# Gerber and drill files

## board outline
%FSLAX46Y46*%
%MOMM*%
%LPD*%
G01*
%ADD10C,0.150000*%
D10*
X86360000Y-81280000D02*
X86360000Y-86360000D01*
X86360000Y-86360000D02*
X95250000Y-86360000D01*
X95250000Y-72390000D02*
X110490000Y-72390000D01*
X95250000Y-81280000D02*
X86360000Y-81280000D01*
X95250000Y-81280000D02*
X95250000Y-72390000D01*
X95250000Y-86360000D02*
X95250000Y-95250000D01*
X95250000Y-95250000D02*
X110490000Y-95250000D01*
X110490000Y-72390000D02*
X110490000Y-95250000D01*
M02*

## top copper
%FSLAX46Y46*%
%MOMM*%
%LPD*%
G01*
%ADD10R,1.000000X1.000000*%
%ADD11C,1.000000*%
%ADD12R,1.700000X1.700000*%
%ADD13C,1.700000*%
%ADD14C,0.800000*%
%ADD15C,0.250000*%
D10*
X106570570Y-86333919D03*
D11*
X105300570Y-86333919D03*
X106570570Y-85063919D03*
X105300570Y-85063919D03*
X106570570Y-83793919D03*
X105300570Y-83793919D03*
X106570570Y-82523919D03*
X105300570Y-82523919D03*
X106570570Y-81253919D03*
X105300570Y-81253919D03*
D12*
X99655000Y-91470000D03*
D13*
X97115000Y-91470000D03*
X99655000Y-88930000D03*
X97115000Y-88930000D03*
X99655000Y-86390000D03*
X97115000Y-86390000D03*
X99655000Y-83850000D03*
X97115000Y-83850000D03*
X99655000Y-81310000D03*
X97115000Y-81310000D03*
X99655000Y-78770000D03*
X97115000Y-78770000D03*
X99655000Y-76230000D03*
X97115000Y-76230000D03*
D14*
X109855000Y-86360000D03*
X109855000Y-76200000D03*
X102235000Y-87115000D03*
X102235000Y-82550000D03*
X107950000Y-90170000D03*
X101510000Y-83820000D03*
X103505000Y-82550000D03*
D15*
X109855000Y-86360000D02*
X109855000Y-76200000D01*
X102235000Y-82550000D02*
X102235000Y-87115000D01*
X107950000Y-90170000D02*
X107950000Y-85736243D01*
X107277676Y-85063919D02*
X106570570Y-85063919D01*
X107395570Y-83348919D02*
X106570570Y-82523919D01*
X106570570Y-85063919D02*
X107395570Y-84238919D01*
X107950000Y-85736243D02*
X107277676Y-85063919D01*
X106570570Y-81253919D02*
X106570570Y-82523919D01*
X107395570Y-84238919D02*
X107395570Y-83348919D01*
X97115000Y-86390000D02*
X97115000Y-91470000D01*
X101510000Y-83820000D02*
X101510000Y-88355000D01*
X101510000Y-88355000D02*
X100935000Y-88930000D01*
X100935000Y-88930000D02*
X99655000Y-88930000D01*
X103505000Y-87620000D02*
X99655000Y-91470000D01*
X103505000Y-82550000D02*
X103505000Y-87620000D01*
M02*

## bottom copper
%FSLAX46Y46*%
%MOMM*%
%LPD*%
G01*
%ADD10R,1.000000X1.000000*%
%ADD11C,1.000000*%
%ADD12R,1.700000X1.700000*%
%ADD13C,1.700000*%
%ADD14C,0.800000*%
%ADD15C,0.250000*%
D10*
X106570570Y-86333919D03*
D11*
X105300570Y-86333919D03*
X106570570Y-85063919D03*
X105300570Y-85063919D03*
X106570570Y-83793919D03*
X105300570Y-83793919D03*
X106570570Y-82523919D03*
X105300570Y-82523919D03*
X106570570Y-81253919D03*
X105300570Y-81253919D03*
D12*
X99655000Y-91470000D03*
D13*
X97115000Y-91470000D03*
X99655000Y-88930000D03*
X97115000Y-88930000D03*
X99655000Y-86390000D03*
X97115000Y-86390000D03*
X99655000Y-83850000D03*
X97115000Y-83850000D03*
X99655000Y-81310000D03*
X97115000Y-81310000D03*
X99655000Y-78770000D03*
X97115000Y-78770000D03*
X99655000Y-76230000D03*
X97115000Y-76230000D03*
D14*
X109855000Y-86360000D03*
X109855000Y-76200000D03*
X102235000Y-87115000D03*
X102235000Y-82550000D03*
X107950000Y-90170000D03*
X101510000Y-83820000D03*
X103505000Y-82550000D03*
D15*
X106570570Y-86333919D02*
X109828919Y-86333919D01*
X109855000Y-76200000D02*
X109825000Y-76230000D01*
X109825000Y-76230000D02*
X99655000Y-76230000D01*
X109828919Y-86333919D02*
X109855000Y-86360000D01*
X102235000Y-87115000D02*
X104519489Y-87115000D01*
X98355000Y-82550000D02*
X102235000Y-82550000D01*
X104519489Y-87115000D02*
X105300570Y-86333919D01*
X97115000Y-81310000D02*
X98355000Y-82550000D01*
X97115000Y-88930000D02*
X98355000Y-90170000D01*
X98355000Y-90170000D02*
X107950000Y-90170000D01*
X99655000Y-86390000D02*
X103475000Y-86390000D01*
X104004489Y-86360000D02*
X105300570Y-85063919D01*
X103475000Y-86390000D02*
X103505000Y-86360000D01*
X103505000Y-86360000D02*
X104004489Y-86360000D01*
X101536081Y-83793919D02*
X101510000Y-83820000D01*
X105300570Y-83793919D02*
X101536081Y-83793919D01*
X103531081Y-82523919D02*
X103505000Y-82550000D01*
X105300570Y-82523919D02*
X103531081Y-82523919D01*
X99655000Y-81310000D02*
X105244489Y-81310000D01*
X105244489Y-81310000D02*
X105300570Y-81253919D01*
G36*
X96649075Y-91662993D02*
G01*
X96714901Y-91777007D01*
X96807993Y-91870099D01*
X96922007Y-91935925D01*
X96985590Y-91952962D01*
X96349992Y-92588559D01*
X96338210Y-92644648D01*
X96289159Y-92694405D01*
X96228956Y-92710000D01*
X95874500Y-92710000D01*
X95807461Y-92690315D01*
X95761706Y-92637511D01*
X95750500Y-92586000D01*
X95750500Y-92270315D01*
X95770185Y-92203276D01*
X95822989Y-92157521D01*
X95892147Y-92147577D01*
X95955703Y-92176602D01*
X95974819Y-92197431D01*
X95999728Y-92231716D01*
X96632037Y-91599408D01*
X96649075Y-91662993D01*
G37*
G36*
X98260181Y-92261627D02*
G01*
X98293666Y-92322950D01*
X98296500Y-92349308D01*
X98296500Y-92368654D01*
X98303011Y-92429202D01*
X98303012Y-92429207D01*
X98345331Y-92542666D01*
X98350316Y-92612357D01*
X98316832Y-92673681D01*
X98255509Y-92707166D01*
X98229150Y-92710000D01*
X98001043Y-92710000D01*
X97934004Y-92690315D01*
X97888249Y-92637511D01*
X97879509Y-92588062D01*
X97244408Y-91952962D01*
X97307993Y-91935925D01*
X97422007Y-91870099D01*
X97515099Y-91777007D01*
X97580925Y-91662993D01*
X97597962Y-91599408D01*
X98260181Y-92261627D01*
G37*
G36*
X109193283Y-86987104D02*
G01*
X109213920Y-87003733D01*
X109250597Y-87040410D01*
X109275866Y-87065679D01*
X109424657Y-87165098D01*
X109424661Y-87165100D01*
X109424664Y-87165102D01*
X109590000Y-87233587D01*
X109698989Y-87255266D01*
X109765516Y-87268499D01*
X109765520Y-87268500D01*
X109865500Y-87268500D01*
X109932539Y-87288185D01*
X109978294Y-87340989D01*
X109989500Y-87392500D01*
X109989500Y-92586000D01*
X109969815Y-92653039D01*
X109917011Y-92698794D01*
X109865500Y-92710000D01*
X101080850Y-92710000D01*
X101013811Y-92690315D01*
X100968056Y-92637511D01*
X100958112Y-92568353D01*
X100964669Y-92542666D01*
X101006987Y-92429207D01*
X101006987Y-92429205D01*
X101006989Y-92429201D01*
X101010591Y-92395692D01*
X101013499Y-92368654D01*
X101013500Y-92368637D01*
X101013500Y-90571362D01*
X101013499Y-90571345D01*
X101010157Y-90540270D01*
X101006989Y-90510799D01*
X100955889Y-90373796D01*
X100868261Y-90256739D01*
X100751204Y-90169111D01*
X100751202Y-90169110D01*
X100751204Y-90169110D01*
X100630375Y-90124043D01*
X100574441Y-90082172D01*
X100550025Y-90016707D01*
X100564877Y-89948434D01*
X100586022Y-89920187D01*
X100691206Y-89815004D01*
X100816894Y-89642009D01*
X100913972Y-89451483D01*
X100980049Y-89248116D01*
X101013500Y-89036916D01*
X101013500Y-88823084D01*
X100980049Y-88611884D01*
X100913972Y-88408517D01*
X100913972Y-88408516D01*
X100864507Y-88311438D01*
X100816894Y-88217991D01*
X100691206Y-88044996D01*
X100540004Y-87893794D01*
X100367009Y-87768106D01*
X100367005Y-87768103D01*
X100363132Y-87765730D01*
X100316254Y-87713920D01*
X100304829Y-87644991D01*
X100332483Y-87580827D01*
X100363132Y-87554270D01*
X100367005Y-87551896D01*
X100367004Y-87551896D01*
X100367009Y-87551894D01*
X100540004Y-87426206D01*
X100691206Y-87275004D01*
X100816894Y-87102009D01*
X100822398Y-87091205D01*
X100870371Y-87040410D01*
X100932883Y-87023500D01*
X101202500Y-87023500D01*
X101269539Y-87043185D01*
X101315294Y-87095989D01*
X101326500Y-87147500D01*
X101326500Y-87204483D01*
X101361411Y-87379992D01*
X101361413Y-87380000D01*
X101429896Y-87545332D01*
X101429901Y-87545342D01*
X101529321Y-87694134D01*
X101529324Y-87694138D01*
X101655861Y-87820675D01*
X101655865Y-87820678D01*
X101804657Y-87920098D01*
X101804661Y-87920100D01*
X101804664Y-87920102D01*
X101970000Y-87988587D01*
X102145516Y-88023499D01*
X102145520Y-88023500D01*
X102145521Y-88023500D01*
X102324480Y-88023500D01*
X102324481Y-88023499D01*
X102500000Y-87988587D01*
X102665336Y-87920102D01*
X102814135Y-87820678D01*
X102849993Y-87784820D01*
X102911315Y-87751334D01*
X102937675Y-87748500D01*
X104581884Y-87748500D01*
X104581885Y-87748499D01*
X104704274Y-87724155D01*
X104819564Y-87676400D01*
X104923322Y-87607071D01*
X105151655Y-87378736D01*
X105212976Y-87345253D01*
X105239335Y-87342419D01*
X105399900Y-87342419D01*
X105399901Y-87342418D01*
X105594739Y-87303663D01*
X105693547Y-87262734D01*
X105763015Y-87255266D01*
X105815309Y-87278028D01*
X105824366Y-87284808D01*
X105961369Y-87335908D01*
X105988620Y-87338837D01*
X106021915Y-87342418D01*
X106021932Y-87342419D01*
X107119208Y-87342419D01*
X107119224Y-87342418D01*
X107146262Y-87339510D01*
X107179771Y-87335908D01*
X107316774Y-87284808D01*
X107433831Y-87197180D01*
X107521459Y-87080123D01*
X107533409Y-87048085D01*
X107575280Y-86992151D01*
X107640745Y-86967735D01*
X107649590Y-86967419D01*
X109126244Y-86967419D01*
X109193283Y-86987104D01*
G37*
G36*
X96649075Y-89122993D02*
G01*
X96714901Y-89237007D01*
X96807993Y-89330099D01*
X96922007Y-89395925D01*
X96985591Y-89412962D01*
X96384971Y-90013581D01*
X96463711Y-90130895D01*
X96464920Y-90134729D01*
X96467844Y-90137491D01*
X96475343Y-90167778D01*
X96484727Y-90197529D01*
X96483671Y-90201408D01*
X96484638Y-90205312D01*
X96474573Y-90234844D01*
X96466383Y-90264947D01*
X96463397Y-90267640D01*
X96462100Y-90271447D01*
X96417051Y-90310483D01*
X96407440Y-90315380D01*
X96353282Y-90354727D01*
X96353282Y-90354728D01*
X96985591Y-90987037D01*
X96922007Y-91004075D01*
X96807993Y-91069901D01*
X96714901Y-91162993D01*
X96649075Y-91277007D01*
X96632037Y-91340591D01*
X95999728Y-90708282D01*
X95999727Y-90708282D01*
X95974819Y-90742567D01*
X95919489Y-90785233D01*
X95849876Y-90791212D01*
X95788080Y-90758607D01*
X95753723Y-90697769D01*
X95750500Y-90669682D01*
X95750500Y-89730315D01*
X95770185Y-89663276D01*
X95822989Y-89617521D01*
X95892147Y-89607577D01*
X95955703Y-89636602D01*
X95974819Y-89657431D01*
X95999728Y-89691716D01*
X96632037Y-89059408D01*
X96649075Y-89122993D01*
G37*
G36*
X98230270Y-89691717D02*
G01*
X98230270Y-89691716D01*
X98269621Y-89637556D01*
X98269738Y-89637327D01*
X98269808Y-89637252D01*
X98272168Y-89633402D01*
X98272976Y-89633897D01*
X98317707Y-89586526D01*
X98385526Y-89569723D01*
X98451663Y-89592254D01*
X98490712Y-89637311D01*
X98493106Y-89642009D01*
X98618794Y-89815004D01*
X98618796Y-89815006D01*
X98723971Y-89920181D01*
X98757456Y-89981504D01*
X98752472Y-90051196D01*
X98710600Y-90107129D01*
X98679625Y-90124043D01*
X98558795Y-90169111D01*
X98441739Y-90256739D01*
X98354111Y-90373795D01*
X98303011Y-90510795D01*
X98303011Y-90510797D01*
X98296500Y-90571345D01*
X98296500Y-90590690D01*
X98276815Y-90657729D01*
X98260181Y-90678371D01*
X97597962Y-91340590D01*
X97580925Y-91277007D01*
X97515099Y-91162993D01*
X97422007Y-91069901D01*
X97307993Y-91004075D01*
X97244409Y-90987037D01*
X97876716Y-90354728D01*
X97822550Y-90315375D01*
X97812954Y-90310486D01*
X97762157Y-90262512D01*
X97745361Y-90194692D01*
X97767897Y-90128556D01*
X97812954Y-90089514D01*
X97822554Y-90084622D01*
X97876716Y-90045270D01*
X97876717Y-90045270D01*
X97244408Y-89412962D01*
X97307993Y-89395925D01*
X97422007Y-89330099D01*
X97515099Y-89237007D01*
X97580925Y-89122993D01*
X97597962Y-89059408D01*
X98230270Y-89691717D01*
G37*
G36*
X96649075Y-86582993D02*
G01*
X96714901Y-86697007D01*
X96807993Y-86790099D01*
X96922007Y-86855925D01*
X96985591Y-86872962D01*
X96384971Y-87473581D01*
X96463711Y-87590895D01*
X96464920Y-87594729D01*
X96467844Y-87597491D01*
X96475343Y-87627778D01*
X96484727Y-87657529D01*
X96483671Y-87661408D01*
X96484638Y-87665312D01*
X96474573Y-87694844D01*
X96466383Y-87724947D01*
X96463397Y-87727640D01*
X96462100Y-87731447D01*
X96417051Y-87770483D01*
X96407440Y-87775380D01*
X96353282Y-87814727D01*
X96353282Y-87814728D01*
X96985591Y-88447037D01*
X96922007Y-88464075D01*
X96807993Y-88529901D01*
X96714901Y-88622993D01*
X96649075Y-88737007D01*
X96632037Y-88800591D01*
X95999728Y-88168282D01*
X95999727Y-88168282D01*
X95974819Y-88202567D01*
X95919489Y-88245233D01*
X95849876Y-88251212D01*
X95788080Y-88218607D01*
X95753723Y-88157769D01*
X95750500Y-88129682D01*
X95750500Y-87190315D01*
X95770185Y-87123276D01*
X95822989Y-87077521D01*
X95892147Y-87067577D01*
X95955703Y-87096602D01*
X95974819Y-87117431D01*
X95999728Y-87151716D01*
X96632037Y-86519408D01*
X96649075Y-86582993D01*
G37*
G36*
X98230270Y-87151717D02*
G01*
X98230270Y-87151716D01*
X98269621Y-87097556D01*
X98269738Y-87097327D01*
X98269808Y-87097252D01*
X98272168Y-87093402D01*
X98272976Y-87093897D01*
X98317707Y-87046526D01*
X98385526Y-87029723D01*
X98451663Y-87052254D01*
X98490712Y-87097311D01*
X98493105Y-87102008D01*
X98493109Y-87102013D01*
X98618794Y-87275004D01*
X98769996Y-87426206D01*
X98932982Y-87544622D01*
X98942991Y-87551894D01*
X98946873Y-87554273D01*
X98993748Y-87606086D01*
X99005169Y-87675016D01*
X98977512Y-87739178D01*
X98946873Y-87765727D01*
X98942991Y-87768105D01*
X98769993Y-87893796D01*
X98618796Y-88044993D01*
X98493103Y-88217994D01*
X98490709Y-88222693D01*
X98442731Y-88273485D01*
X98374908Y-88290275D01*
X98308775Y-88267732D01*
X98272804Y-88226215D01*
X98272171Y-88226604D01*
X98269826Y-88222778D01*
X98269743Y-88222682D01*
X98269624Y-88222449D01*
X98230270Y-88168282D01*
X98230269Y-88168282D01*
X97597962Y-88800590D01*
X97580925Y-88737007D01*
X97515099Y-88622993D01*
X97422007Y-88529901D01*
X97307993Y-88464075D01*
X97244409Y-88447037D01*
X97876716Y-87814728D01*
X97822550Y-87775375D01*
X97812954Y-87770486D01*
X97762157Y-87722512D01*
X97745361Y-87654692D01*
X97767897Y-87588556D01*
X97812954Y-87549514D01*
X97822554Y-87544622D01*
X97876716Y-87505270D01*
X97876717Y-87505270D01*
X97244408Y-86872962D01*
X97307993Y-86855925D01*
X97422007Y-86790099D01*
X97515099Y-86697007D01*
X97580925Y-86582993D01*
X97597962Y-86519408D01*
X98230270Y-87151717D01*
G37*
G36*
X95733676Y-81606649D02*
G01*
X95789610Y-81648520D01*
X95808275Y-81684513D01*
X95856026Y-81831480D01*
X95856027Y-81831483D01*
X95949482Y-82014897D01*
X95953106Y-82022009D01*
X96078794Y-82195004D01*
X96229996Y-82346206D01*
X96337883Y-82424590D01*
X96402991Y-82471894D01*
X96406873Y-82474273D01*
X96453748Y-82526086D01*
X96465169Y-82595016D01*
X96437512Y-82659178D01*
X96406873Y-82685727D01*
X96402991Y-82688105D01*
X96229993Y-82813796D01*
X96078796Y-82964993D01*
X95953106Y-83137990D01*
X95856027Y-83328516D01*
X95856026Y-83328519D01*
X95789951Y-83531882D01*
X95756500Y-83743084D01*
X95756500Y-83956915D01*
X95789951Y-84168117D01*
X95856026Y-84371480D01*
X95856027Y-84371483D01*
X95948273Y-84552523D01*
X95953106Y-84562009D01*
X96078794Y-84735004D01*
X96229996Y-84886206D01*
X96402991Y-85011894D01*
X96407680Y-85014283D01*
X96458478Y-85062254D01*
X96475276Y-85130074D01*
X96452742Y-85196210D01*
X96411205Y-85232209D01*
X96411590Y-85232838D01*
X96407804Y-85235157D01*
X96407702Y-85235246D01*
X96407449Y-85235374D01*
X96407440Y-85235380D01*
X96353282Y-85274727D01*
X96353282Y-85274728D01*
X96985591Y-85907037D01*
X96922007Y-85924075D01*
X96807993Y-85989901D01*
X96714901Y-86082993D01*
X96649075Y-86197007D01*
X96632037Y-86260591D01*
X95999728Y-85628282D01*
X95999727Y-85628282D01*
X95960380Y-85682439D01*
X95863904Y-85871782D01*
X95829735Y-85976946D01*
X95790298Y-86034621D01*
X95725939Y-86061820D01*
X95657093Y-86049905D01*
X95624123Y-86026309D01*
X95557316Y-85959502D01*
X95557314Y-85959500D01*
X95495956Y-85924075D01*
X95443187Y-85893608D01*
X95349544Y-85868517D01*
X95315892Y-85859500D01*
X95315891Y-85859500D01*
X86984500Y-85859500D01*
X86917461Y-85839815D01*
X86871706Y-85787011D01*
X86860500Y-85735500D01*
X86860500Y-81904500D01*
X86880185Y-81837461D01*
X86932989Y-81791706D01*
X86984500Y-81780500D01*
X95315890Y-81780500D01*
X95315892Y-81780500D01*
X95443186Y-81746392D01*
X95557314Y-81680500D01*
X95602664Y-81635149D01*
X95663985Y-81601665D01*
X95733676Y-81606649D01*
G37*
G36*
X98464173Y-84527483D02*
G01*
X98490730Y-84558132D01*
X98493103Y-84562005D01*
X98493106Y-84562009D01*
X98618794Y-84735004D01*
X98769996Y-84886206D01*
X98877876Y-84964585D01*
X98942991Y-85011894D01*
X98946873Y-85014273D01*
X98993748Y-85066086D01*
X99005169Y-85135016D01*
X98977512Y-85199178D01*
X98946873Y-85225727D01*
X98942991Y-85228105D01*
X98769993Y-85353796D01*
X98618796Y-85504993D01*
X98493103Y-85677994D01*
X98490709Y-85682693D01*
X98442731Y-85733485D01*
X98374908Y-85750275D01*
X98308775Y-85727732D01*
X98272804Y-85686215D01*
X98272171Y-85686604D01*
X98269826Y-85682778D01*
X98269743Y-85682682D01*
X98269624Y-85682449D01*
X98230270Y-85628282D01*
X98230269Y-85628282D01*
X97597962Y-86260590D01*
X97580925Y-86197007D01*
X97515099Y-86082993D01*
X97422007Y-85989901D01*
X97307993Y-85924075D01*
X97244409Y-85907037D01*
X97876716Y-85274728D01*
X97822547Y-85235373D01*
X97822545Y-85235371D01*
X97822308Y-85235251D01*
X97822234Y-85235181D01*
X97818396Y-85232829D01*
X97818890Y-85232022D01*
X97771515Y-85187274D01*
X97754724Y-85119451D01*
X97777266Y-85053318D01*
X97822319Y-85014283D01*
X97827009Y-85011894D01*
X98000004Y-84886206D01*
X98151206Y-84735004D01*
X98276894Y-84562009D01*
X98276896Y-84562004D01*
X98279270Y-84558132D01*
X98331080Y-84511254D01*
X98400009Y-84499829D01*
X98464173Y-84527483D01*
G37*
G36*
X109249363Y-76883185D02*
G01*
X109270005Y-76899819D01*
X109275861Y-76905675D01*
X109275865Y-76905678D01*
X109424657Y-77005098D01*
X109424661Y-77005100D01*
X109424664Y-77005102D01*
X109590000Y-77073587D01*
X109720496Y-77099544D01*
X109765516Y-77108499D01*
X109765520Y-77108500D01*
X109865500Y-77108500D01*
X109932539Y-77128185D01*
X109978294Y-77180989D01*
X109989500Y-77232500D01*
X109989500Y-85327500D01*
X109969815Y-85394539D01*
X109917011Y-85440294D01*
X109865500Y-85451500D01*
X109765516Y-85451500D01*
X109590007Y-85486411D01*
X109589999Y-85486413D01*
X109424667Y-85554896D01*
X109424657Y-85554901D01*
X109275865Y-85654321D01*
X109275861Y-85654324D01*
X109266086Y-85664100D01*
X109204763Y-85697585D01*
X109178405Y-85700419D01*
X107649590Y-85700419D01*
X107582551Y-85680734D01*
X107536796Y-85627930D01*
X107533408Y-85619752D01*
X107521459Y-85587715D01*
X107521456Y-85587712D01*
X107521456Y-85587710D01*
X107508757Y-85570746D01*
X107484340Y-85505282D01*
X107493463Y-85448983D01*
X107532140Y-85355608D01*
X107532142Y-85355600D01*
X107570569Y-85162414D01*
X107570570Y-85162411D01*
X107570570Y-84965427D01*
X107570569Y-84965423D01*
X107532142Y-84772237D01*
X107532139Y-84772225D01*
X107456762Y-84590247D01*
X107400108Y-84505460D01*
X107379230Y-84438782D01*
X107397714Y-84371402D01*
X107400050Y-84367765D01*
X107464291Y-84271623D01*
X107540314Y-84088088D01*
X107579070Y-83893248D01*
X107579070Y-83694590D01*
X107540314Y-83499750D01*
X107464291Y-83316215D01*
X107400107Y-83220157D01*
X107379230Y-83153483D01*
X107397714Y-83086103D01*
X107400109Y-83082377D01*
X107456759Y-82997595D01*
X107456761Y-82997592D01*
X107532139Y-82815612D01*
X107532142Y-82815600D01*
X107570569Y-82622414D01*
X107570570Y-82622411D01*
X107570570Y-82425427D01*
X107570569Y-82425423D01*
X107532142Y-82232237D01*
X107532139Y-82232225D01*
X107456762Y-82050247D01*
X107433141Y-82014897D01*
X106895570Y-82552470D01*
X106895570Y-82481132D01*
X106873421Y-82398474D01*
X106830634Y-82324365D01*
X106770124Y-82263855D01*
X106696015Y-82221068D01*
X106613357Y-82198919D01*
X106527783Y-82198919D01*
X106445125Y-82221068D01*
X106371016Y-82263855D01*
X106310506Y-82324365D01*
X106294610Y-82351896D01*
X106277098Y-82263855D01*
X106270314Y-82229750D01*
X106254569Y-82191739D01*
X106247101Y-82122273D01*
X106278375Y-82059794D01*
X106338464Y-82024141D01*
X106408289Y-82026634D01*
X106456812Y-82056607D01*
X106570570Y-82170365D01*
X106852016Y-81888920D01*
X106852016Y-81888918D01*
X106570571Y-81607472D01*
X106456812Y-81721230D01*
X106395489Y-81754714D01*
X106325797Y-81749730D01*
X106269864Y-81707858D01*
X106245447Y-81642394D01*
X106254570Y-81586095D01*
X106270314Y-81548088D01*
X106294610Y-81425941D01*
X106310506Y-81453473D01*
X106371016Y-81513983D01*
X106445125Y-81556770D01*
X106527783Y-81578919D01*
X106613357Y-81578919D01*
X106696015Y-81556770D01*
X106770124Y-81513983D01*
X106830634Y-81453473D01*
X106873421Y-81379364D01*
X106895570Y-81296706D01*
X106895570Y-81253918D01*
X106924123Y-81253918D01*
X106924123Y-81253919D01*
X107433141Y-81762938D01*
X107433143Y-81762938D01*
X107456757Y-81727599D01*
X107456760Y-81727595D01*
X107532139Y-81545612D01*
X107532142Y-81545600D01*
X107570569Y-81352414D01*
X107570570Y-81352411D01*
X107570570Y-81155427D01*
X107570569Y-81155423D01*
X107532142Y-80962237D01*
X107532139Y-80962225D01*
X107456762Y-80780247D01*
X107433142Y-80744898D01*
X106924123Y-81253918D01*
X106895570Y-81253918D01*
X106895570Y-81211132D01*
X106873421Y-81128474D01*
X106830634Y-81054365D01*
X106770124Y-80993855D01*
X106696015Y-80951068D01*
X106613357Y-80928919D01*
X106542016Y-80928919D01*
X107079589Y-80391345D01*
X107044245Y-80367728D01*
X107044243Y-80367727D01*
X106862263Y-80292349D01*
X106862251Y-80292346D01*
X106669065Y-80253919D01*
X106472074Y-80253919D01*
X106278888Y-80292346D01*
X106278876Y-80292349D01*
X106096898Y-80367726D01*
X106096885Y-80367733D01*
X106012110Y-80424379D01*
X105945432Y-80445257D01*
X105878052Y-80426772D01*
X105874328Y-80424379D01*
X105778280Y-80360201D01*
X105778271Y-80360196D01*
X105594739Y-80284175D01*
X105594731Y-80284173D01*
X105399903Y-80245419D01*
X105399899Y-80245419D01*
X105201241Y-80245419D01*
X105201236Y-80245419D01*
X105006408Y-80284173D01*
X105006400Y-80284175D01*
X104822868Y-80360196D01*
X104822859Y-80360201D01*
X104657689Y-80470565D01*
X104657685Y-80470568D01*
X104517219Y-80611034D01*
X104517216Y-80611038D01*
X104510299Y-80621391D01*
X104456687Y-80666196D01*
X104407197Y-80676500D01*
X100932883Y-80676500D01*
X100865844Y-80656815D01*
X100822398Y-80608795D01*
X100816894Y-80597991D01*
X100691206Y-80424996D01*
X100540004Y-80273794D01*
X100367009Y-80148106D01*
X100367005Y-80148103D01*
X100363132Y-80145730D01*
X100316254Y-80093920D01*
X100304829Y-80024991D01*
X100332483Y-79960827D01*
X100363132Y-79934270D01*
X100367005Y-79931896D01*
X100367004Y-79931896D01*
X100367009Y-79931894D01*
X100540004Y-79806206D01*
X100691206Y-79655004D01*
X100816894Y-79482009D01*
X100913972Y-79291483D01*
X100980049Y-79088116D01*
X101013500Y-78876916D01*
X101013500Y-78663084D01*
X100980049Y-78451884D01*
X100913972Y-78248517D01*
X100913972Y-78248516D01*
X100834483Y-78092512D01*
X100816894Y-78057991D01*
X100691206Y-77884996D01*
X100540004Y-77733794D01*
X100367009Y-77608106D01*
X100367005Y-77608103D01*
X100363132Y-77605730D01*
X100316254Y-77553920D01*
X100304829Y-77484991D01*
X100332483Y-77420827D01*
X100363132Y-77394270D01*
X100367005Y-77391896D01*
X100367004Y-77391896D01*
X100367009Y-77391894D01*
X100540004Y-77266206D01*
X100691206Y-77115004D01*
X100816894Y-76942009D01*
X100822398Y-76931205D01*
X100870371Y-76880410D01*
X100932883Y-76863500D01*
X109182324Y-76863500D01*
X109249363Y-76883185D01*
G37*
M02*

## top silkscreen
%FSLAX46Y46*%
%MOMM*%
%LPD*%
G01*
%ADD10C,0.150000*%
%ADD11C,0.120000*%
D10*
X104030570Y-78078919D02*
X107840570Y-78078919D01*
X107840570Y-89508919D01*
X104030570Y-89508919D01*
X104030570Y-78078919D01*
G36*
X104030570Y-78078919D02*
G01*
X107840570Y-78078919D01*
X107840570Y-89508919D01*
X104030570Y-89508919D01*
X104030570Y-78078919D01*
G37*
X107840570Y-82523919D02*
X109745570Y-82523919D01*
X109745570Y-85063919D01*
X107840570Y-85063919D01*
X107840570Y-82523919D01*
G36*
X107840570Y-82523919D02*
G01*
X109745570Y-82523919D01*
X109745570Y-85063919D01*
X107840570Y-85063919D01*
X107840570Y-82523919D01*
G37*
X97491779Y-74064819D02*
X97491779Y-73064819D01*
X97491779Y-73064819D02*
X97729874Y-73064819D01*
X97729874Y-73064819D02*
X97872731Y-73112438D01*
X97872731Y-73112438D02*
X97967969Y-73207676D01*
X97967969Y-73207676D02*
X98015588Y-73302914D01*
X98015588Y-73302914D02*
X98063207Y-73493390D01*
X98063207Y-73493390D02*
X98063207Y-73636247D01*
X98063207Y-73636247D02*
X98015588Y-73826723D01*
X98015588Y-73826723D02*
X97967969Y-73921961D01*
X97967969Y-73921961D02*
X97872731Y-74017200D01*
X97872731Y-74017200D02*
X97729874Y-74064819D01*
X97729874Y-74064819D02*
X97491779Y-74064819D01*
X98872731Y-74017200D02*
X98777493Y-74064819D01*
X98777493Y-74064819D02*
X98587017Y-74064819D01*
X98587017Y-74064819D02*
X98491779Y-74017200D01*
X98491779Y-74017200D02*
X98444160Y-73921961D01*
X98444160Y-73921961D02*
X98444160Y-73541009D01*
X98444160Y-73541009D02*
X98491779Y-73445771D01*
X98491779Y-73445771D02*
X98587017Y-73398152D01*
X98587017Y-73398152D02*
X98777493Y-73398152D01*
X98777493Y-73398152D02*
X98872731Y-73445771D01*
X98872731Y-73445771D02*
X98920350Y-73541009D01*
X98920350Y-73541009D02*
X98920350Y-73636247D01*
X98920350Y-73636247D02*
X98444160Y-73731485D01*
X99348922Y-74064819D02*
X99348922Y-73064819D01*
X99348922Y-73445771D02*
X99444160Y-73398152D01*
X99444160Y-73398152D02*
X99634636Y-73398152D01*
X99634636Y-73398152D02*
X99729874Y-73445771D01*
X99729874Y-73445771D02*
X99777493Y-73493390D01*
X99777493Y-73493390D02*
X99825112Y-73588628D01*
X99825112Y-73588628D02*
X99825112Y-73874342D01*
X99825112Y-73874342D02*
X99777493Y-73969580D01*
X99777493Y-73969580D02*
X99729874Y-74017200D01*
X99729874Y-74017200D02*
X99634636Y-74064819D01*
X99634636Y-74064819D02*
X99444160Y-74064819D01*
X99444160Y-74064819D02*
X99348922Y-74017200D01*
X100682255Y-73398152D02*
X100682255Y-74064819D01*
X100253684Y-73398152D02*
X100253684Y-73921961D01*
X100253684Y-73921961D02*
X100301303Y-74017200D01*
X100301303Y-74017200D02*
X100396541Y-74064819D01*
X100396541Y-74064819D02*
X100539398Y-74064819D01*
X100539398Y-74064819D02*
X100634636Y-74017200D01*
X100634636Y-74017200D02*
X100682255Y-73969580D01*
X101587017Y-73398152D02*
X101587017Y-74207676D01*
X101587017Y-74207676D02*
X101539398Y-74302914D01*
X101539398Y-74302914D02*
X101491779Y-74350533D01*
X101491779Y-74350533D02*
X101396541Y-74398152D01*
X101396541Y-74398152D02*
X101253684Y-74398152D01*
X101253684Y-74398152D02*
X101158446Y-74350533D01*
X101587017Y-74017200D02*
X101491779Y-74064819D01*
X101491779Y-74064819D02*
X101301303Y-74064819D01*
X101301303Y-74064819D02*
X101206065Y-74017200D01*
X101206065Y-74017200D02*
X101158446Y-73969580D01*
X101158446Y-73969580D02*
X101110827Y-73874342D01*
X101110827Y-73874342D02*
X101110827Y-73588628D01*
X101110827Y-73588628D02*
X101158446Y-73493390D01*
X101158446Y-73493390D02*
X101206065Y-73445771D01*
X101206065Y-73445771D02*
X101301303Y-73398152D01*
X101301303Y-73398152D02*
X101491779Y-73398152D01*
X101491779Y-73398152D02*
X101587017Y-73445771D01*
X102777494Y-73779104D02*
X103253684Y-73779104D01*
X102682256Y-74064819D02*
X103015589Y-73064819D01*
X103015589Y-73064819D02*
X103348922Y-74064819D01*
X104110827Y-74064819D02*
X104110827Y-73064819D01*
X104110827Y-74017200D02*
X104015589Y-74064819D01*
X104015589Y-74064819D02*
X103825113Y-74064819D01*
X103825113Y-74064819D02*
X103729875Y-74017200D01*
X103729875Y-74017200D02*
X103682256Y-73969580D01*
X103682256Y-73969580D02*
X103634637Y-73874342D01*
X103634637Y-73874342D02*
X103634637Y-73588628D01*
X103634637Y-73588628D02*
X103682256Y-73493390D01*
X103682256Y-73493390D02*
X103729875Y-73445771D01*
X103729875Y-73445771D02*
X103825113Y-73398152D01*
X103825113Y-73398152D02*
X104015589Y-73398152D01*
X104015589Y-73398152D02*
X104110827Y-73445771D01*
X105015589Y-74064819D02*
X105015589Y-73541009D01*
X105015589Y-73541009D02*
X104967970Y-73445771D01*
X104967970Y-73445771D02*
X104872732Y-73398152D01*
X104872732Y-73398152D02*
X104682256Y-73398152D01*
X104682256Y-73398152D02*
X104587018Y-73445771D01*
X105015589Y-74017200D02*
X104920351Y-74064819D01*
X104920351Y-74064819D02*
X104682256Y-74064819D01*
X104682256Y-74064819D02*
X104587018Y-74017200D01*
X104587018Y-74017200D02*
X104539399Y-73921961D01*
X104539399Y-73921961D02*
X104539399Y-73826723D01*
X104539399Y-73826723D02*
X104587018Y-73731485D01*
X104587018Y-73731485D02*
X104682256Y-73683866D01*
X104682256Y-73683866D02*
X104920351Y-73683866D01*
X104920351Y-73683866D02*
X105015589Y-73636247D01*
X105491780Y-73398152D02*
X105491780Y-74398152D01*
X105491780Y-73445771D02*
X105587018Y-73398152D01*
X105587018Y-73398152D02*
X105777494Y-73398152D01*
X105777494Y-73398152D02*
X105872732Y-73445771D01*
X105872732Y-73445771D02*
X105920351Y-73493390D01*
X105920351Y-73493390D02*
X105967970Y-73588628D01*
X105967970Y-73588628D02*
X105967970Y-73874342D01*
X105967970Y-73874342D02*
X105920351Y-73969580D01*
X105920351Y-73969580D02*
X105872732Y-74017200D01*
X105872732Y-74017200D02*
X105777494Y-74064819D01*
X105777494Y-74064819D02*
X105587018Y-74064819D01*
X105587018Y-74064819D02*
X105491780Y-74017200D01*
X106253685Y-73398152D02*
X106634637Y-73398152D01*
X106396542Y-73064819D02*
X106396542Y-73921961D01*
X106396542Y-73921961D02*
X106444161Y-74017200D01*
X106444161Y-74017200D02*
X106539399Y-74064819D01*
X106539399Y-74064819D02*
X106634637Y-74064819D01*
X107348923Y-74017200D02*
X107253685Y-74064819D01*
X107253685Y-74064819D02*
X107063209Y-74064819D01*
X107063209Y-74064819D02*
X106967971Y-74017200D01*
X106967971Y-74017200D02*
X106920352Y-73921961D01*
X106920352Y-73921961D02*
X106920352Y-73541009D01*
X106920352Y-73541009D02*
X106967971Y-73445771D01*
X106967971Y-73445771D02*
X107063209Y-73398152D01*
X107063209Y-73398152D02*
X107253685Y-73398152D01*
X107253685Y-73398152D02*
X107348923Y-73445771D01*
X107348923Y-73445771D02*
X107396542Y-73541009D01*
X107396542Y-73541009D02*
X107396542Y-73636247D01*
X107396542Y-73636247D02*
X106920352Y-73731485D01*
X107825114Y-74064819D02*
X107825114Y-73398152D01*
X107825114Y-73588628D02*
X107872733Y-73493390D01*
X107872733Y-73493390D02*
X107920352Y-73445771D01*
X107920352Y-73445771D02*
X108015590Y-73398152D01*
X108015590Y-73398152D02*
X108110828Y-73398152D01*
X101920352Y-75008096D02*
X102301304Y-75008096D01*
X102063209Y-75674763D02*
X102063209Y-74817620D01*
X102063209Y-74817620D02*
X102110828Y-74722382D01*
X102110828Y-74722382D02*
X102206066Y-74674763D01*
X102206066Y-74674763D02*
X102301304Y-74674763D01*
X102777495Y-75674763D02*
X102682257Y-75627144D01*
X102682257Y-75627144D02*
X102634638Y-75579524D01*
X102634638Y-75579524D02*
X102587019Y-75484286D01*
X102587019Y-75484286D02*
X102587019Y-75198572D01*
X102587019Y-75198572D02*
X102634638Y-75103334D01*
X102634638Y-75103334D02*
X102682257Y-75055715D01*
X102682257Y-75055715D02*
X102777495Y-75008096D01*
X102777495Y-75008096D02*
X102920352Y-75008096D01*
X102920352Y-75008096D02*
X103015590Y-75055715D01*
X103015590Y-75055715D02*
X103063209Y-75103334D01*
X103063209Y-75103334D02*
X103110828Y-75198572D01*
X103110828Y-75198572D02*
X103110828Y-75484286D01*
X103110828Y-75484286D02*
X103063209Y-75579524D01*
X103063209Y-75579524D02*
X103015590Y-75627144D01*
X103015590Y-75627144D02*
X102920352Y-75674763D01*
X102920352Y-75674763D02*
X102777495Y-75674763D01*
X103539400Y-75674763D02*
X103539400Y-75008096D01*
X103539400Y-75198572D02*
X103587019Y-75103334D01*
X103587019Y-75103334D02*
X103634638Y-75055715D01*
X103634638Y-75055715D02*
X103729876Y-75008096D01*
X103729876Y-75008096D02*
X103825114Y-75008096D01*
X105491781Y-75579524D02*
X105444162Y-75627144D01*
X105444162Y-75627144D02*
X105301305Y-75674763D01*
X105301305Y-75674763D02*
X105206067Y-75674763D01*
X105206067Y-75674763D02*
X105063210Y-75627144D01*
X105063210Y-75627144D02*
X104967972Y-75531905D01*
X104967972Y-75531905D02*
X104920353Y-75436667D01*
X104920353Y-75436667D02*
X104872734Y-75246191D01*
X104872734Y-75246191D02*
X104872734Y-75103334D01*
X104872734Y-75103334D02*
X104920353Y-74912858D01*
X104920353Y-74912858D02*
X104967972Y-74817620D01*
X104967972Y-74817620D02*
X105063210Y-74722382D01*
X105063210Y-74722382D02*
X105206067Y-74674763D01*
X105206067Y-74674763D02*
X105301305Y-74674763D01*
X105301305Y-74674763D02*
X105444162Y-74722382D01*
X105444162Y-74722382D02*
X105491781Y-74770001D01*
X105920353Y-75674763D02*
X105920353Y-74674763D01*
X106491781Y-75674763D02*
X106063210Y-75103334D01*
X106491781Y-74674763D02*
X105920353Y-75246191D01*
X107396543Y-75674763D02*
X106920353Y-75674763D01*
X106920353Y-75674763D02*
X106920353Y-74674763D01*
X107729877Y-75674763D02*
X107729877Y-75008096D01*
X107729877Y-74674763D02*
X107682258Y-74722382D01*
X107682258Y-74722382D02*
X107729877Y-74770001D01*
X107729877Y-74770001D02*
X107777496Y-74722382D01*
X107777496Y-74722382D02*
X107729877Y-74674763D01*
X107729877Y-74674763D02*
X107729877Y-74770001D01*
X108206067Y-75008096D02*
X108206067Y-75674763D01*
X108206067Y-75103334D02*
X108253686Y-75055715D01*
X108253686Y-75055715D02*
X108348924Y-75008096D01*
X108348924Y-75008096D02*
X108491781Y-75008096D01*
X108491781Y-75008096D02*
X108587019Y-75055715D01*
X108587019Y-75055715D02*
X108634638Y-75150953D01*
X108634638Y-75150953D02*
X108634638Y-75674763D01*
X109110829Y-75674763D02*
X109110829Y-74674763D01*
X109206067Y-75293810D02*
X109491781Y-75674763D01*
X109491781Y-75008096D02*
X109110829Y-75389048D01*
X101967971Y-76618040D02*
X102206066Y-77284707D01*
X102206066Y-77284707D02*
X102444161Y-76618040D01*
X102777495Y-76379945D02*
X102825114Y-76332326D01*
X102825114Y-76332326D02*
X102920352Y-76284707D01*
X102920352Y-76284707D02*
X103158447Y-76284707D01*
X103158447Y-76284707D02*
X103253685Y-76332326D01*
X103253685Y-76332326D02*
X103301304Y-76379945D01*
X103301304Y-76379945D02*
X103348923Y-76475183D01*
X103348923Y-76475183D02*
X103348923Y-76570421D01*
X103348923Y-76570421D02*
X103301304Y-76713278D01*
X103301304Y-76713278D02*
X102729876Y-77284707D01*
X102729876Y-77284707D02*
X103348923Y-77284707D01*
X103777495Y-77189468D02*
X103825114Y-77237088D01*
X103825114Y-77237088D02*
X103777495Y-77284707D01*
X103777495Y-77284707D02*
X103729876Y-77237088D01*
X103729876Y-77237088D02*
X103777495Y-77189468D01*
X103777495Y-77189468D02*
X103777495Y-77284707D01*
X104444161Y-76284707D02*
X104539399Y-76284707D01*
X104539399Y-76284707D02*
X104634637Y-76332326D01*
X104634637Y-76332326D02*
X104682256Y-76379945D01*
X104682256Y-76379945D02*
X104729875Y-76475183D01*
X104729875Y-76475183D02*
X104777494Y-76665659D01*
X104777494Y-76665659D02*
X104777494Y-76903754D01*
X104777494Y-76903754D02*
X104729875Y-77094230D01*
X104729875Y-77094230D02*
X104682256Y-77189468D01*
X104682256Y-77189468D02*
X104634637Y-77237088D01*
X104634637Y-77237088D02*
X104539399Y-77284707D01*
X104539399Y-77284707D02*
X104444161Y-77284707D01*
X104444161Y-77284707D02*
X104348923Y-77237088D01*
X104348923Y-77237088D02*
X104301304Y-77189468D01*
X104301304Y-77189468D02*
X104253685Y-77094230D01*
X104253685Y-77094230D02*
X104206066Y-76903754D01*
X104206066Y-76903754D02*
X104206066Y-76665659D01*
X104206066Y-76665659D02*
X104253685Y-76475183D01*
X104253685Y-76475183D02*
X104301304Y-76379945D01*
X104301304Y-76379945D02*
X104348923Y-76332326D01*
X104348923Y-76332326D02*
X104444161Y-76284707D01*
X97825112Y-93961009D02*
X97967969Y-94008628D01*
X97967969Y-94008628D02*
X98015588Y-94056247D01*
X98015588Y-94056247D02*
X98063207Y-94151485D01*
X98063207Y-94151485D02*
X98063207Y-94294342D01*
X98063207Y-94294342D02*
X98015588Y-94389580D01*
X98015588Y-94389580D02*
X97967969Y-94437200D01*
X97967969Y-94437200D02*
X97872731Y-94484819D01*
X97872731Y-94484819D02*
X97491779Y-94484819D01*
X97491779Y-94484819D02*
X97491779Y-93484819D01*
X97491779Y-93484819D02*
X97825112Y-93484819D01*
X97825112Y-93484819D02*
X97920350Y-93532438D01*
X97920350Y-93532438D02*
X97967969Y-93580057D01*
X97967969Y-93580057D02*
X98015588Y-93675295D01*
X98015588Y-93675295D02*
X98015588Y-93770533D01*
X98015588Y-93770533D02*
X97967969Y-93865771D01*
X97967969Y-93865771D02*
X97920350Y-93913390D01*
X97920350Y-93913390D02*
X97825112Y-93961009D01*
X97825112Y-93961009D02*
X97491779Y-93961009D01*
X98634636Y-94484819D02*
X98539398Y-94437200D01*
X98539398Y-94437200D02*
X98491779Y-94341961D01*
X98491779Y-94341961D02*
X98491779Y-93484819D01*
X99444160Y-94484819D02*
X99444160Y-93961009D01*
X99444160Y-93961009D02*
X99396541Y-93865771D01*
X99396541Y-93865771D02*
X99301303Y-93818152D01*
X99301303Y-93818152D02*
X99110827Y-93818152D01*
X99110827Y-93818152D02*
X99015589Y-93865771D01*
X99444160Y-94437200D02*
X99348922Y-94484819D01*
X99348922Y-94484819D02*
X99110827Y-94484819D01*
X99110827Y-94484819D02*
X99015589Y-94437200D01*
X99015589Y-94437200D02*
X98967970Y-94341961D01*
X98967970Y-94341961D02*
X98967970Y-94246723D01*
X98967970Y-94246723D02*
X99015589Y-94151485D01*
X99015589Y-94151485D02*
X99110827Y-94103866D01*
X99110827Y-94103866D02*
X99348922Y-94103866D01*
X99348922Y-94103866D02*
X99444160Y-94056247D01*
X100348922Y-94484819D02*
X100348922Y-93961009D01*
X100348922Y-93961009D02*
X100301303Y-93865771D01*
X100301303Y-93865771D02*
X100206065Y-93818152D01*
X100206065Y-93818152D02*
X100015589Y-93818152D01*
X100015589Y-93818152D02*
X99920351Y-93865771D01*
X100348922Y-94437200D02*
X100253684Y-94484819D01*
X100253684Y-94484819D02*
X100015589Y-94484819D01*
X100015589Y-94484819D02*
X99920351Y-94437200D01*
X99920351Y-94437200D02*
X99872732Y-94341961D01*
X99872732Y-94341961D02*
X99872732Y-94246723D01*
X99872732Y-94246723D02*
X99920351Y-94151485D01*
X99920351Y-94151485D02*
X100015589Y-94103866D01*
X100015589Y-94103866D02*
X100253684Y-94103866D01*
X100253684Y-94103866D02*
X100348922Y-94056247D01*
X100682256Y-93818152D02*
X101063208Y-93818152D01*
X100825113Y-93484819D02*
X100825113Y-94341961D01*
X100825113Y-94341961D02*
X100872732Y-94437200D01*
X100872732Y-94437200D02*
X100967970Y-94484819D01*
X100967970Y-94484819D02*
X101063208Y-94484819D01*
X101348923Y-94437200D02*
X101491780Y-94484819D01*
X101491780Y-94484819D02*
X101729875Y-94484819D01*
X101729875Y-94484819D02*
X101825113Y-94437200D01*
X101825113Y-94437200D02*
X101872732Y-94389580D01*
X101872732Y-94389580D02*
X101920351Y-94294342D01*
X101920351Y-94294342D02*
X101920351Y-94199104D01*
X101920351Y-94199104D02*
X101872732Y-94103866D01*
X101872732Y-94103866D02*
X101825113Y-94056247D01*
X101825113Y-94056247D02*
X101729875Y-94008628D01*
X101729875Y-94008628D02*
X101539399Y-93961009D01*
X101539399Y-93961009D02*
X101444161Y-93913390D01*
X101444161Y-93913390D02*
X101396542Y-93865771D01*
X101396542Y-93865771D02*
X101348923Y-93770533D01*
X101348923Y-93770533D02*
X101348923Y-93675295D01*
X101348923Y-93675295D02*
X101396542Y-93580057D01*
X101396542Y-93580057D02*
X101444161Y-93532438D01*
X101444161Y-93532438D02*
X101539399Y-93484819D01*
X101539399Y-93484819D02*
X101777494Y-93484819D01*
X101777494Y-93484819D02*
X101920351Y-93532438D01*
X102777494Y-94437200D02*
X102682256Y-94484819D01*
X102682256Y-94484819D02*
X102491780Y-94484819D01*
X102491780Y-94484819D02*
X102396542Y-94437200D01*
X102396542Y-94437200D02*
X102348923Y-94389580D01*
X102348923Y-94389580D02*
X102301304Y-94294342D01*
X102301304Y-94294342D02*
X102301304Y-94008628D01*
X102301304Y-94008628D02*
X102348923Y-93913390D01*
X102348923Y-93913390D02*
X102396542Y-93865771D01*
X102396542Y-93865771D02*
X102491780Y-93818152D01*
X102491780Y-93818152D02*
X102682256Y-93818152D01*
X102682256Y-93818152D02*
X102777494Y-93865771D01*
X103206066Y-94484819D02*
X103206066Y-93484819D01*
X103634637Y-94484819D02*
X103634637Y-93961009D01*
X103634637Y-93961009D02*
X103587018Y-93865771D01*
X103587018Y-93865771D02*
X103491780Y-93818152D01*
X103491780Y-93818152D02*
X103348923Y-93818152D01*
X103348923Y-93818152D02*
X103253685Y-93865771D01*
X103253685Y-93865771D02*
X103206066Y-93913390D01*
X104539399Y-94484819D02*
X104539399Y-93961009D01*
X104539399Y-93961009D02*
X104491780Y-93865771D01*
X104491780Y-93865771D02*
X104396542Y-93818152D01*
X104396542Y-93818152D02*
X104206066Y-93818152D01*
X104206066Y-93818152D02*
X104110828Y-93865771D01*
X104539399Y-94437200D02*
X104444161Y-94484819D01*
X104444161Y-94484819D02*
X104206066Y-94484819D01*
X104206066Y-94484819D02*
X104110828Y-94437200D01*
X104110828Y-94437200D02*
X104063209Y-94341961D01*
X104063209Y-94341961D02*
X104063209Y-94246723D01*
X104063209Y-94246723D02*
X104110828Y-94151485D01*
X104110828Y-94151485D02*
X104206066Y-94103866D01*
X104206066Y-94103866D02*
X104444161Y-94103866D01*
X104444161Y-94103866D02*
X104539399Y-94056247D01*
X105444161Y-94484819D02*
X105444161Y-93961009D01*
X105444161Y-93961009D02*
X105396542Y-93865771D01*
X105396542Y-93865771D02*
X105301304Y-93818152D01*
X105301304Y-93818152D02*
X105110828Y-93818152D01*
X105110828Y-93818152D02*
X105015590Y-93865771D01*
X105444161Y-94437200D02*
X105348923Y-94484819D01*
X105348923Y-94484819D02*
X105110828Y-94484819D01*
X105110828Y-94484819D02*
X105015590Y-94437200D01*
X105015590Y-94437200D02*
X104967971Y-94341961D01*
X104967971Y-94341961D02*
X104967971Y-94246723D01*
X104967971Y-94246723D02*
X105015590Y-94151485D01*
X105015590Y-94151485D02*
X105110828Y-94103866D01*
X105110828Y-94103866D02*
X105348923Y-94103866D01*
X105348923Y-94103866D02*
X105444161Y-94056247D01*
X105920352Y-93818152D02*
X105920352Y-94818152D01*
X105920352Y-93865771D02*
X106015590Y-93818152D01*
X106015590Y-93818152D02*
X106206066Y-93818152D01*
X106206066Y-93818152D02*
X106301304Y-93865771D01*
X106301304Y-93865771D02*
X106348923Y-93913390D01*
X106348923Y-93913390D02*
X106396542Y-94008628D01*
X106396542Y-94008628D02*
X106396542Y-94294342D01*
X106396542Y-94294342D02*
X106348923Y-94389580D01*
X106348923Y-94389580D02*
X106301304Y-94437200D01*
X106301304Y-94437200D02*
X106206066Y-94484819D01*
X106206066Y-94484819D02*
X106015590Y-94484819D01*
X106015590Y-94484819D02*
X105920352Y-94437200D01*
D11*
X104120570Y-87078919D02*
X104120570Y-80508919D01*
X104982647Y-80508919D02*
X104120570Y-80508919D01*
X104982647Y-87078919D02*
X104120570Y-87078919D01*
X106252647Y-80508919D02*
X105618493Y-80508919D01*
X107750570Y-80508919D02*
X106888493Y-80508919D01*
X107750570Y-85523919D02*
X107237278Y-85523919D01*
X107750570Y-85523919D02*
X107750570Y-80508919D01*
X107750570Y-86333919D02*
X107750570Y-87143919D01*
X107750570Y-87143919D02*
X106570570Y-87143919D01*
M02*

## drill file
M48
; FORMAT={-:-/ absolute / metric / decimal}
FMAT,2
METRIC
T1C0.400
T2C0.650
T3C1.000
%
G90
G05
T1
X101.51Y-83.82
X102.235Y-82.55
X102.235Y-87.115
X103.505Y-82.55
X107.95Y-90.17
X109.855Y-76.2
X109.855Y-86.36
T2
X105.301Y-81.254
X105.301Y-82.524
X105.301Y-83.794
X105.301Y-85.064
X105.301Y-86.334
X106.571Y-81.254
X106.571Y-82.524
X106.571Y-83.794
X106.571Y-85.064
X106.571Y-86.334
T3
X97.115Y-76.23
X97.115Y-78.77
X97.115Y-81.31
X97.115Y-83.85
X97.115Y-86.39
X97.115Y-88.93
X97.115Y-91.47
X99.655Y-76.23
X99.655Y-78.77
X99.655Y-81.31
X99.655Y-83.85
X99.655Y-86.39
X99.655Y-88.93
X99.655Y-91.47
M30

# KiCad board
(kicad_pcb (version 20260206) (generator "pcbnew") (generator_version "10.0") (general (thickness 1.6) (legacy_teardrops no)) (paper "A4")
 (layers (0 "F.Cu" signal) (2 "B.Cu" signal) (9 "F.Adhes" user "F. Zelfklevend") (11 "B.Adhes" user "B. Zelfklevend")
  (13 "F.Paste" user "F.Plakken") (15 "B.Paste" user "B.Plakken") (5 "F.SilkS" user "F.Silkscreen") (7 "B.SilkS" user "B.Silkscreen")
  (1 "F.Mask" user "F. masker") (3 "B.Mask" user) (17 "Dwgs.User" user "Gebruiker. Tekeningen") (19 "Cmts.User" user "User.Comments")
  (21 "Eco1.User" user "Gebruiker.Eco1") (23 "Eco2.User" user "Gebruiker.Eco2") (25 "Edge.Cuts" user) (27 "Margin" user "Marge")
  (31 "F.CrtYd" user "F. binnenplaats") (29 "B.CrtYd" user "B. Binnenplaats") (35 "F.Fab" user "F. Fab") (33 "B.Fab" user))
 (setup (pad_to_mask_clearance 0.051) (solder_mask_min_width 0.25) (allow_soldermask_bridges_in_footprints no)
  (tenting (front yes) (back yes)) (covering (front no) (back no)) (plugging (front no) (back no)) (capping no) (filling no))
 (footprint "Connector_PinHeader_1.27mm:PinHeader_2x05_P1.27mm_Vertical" (layer "F.Cu") (at 106.57057 86.333919 180)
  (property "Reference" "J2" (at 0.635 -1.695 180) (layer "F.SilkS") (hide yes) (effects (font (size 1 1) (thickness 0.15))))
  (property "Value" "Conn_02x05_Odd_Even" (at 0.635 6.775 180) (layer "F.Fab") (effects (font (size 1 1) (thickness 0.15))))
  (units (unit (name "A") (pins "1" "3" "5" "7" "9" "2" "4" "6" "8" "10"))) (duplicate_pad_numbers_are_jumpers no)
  (fp_line (start 2.45 -0.745) (end 2.45 5.825) (stroke (width 0.12) (type solid)) (layer "F.SilkS"))
  (fp_line (start 1.587923 5.825) (end 2.45 5.825) (stroke (width 0.12) (type solid)) (layer "F.SilkS"))
  (fp_line (start 1.587923 -0.745) (end 2.45 -0.745) (stroke (width 0.12) (type solid)) (layer "F.SilkS"))
  (fp_line (start 0.317923 5.825) (end 0.952077 5.825) (stroke (width 0.12) (type solid)) (layer "F.SilkS"))
  (fp_line (start -1.18 5.825) (end -0.317923 5.825) (stroke (width 0.12) (type solid)) (layer "F.SilkS"))
  (fp_line (start -1.18 0.81) (end -0.666708 0.81) (stroke (width 0.12) (type solid)) (layer "F.SilkS"))
  (fp_line (start -1.18 0.81) (end -1.18 5.825) (stroke (width 0.12) (type solid)) (layer "F.SilkS"))
  (fp_line (start -1.18 0) (end -1.18 -0.81) (stroke (width 0.12) (type solid)) (layer "F.SilkS"))
  (fp_line (start -1.18 -0.81) (end 0 -0.81) (stroke (width 0.12) (type solid)) (layer "F.SilkS"))
  (pad "1" thru_hole rect (at 0 0 180) (size 1 1) (drill 0.65) (layers "*.Cu" "*.Mask") (remove_unused_layers no) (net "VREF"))
  (pad "2" thru_hole circle (at 1.27 0 180) (size 1 1) (drill 0.65) (layers "*.Cu" "*.Mask") (remove_unused_layers no) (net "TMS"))
  (pad "3" thru_hole circle (at 0 1.27 180) (size 1 1) (drill 0.65) (layers "*.Cu" "*.Mask") (remove_unused_layers no) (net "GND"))
  (pad "4" thru_hole circle (at 1.27 1.27 180) (size 1 1) (drill 0.65) (layers "*.Cu" "*.Mask") (remove_unused_layers no) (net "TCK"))
  (pad "5" thru_hole circle (at 0 2.54 180) (size 1 1) (drill 0.65) (layers "*.Cu" "*.Mask") (remove_unused_layers no)
   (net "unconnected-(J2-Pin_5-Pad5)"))
  (pad "6" thru_hole circle (at 1.27 2.54 180) (size 1 1) (drill 0.65) (layers "*.Cu" "*.Mask") (remove_unused_layers no) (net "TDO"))
  (pad "7" thru_hole circle (at 0 3.81 180) (size 1 1) (drill 0.65) (layers "*.Cu" "*.Mask") (remove_unused_layers no) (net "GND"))
  (pad "8" thru_hole circle (at 1.27 3.81 180) (size 1 1) (drill 0.65) (layers "*.Cu" "*.Mask") (remove_unused_layers no) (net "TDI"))
  (pad "9" thru_hole circle (at 0 5.08 180) (size 1 1) (drill 0.65) (layers "*.Cu" "*.Mask") (remove_unused_layers no) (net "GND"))
  (pad "10" thru_hole circle (at 1.27 5.08 180) (size 1 1) (drill 0.65) (layers "*.Cu" "*.Mask") (remove_unused_layers no) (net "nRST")))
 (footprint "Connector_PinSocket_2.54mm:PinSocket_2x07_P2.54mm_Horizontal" (layer "B.Cu") (at 99.655 91.47)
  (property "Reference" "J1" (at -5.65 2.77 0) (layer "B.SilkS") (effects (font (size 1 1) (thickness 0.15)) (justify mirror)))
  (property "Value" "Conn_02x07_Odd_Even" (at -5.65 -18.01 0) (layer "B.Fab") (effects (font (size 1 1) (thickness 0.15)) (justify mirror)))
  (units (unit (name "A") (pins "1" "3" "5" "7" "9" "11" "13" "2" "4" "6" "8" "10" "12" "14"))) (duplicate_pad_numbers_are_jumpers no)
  (pad "1" thru_hole rect (at 0 0) (size 1.7 1.7) (drill 1) (layers "*.Cu" "*.Mask") (remove_unused_layers no) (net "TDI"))
  (pad "2" thru_hole circle (at -2.54 0) (size 1.7 1.7) (drill 1) (layers "*.Cu" "*.Mask") (remove_unused_layers no) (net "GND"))
  (pad "3" thru_hole circle (at 0 -2.54) (size 1.7 1.7) (drill 1) (layers "*.Cu" "*.Mask") (remove_unused_layers no) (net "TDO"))
  (pad "4" thru_hole circle (at -2.54 -2.54) (size 1.7 1.7) (drill 1) (layers "*.Cu" "*.Mask") (remove_unused_layers no) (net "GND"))
  (pad "5" thru_hole circle (at 0 -5.08) (size 1.7 1.7) (drill 1) (layers "*.Cu" "*.Mask") (remove_unused_layers no) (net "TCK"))
  (pad "6" thru_hole circle (at -2.54 -5.08) (size 1.7 1.7) (drill 1) (layers "*.Cu" "*.Mask") (remove_unused_layers no) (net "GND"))
  (pad "7" thru_hole circle (at 0 -7.62) (size 1.7 1.7) (drill 1) (layers "*.Cu" "*.Mask") (remove_unused_layers no)
   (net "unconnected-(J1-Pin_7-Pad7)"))
  (pad "8" thru_hole circle (at -2.54 -7.62) (size 1.7 1.7) (drill 1) (layers "*.Cu" "*.Mask") (remove_unused_layers no)
   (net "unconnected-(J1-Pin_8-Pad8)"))
  (pad "9" thru_hole circle (at 0 -10.16) (size 1.7 1.7) (drill 1) (layers "*.Cu" "*.Mask") (remove_unused_layers no) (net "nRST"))
  (pad "10" thru_hole circle (at -2.54 -10.16) (size 1.7 1.7) (drill 1) (layers "*.Cu" "*.Mask") (remove_unused_layers no) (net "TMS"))
  (pad "11" thru_hole circle (at 0 -12.7) (size 1.7 1.7) (drill 1) (layers "*.Cu" "*.Mask") (remove_unused_layers no)
   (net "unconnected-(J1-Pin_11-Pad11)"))
  (pad "12" thru_hole circle (at -2.54 -12.7) (size 1.7 1.7) (drill 1) (layers "*.Cu" "*.Mask") (remove_unused_layers no)
   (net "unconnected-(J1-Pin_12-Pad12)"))
  (pad "13" thru_hole circle (at 0 -15.24) (size 1.7 1.7) (drill 1) (layers "*.Cu" "*.Mask") (remove_unused_layers no) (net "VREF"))
  (pad "14" thru_hole circle (at -2.54 -15.24) (size 1.7 1.7) (drill 1) (layers "*.Cu" "*.Mask") (remove_unused_layers no) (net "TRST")))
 (gr_rect (start 104.03057 78.078919) (end 107.84057 89.508919) (stroke (width 0.15) (type solid)) (fill yes) (layer "F.SilkS"))
 (gr_rect (start 107.84057 82.523919) (end 109.74557 85.063919) (stroke (width 0.15) (type solid)) (fill yes) (layer "F.SilkS"))
 (gr_line (start 86.36 81.28) (end 86.36 86.36) (stroke (width 0.15) (type default)) (layer "Edge.Cuts"))
 (gr_line (start 86.36 86.36) (end 95.25 86.36) (stroke (width 0.15) (type default)) (layer "Edge.Cuts"))
 (gr_line (start 95.25 72.39) (end 110.49 72.39) (stroke (width 0.15) (type default)) (layer "Edge.Cuts"))
 (gr_line (start 95.25 81.28) (end 86.36 81.28) (stroke (width 0.15) (type default)) (layer "Edge.Cuts"))
 (gr_line (start 95.25 81.28) (end 95.25 72.39) (stroke (width 0.15) (type default)) (layer "Edge.Cuts"))
 (gr_line (start 95.25 86.36) (end 95.25 95.25) (stroke (width 0.15) (type default)) (layer "Edge.Cuts"))
 (gr_line (start 95.25 95.25) (end 110.49 95.25) (stroke (width 0.15) (type default)) (layer "Edge.Cuts"))
 (gr_line (start 110.49 72.39) (end 110.49 95.25) (stroke (width 0.15) (type default)) (layer "Edge.Cuts"))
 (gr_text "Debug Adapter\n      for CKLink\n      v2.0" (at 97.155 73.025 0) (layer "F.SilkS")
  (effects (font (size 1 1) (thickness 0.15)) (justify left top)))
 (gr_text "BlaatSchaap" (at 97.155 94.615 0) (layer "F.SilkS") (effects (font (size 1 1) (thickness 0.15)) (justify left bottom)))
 (segment (start 109.855 86.36) (end 109.855 76.2) (width 0.25) (layer "F.Cu") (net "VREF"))
 (via (at 109.855 86.36) (size 0.8) (drill 0.4) (layers "F.Cu" "B.Cu") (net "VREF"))
 (via (at 109.855 76.2) (size 0.8) (drill 0.4) (layers "F.Cu" "B.Cu") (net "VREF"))
 (segment (start 106.57057 86.333919) (end 109.828919 86.333919) (width 0.25) (layer "B.Cu") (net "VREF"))
 (segment (start 109.855 76.2) (end 109.825 76.23) (width 0.25) (layer "B.Cu") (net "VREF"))
 (segment (start 109.825 76.23) (end 99.655 76.23) (width 0.25) (layer "B.Cu") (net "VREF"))
 (segment (start 109.828919 86.333919) (end 109.855 86.36) (width 0.25) (layer "B.Cu") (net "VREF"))
 (segment (start 102.235 82.55) (end 102.235 87.115) (width 0.25) (layer "F.Cu") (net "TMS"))
 (via (at 102.235 87.115) (size 0.8) (drill 0.4) (layers "F.Cu" "B.Cu") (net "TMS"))
 (via (at 102.235 82.55) (size 0.8) (drill 0.4) (layers "F.Cu" "B.Cu") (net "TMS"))
 (segment (start 102.235 87.115) (end 104.519489 87.115) (width 0.25) (layer "B.Cu") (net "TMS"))
 (segment (start 98.355 82.55) (end 102.235 82.55) (width 0.25) (layer "B.Cu") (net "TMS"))
 (segment (start 104.519489 87.115) (end 105.30057 86.333919) (width 0.25) (layer "B.Cu") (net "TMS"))
 (segment (start 97.115 81.31) (end 98.355 82.55) (width 0.25) (layer "B.Cu") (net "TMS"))
 (segment (start 107.95 90.17) (end 107.95 85.736243) (width 0.25) (layer "F.Cu") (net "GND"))
 (segment (start 107.277676 85.063919) (end 106.57057 85.063919) (width 0.25) (layer "F.Cu") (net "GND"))
 (segment (start 107.39557 83.348919) (end 106.57057 82.523919) (width 0.25) (layer "F.Cu") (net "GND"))
 (segment (start 106.57057 85.063919) (end 107.39557 84.238919) (width 0.25) (layer "F.Cu") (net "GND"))
 (segment (start 107.95 85.736243) (end 107.277676 85.063919) (width 0.25) (layer "F.Cu") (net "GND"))
 (segment (start 106.57057 81.253919) (end 106.57057 82.523919) (width 0.25) (layer "F.Cu") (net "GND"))
 (segment (start 107.39557 84.238919) (end 107.39557 83.348919) (width 0.25) (layer "F.Cu") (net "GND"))
 (segment (start 97.115 86.39) (end 97.115 91.47) (width 0.25) (layer "F.Cu") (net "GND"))
 (via (at 107.95 90.17) (size 0.8) (drill 0.4) (layers "F.Cu" "B.Cu") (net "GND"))
 (segment (start 97.115 88.93) (end 98.355 90.17) (width 0.25) (layer "B.Cu") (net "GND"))
 (segment (start 98.355 90.17) (end 107.95 90.17) (width 0.25) (layer "B.Cu") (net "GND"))
 (segment (start 99.655 86.39) (end 103.475 86.39) (width 0.25) (layer "B.Cu") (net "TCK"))
 (segment (start 104.004489 86.36) (end 105.30057 85.063919) (width 0.25) (layer "B.Cu") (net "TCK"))
 (segment (start 103.475 86.39) (end 103.505 86.36) (width 0.25) (layer "B.Cu") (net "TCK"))
 (segment (start 103.505 86.36) (end 104.004489 86.36) (width 0.25) (layer "B.Cu") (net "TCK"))
 (segment (start 101.51 83.82) (end 101.51 88.355) (width 0.25) (layer "F.Cu") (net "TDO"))
 (segment (start 101.51 88.355) (end 100.935 88.93) (width 0.25) (layer "F.Cu") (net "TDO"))
 (segment (start 100.935 88.93) (end 99.655 88.93) (width 0.25) (layer "F.Cu") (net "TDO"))
 (via (at 101.51 83.82) (size 0.8) (drill 0.4) (layers "F.Cu" "B.Cu") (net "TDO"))
 (segment (start 101.536081 83.793919) (end 101.51 83.82) (width 0.25) (layer "B.Cu") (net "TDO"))
 (segment (start 105.30057 83.793919) (end 101.536081 83.793919) (width 0.25) (layer "B.Cu") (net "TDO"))
 (segment (start 103.505 87.62) (end 99.655 91.47) (width 0.25) (layer "F.Cu") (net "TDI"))
 (segment (start 103.505 82.55) (end 103.505 87.62) (width 0.25) (layer "F.Cu") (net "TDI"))
 (via (at 103.505 82.55) (size 0.8) (drill 0.4) (layers "F.Cu" "B.Cu") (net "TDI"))
 (segment (start 103.531081 82.523919) (end 103.505 82.55) (width 0.25) (layer "B.Cu") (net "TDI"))
 (segment (start 105.30057 82.523919) (end 103.531081 82.523919) (width 0.25) (layer "B.Cu") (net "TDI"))
 (segment (start 99.655 81.31) (end 105.244489 81.31) (width 0.25) (layer "B.Cu") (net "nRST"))
 (segment (start 105.244489 81.31) (end 105.30057 81.253919) (width 0.25) (layer "B.Cu") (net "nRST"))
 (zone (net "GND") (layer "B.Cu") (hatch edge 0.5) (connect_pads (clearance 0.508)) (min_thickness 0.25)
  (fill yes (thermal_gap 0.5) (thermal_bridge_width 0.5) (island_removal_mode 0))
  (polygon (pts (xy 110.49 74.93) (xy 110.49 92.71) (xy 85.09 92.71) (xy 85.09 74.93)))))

